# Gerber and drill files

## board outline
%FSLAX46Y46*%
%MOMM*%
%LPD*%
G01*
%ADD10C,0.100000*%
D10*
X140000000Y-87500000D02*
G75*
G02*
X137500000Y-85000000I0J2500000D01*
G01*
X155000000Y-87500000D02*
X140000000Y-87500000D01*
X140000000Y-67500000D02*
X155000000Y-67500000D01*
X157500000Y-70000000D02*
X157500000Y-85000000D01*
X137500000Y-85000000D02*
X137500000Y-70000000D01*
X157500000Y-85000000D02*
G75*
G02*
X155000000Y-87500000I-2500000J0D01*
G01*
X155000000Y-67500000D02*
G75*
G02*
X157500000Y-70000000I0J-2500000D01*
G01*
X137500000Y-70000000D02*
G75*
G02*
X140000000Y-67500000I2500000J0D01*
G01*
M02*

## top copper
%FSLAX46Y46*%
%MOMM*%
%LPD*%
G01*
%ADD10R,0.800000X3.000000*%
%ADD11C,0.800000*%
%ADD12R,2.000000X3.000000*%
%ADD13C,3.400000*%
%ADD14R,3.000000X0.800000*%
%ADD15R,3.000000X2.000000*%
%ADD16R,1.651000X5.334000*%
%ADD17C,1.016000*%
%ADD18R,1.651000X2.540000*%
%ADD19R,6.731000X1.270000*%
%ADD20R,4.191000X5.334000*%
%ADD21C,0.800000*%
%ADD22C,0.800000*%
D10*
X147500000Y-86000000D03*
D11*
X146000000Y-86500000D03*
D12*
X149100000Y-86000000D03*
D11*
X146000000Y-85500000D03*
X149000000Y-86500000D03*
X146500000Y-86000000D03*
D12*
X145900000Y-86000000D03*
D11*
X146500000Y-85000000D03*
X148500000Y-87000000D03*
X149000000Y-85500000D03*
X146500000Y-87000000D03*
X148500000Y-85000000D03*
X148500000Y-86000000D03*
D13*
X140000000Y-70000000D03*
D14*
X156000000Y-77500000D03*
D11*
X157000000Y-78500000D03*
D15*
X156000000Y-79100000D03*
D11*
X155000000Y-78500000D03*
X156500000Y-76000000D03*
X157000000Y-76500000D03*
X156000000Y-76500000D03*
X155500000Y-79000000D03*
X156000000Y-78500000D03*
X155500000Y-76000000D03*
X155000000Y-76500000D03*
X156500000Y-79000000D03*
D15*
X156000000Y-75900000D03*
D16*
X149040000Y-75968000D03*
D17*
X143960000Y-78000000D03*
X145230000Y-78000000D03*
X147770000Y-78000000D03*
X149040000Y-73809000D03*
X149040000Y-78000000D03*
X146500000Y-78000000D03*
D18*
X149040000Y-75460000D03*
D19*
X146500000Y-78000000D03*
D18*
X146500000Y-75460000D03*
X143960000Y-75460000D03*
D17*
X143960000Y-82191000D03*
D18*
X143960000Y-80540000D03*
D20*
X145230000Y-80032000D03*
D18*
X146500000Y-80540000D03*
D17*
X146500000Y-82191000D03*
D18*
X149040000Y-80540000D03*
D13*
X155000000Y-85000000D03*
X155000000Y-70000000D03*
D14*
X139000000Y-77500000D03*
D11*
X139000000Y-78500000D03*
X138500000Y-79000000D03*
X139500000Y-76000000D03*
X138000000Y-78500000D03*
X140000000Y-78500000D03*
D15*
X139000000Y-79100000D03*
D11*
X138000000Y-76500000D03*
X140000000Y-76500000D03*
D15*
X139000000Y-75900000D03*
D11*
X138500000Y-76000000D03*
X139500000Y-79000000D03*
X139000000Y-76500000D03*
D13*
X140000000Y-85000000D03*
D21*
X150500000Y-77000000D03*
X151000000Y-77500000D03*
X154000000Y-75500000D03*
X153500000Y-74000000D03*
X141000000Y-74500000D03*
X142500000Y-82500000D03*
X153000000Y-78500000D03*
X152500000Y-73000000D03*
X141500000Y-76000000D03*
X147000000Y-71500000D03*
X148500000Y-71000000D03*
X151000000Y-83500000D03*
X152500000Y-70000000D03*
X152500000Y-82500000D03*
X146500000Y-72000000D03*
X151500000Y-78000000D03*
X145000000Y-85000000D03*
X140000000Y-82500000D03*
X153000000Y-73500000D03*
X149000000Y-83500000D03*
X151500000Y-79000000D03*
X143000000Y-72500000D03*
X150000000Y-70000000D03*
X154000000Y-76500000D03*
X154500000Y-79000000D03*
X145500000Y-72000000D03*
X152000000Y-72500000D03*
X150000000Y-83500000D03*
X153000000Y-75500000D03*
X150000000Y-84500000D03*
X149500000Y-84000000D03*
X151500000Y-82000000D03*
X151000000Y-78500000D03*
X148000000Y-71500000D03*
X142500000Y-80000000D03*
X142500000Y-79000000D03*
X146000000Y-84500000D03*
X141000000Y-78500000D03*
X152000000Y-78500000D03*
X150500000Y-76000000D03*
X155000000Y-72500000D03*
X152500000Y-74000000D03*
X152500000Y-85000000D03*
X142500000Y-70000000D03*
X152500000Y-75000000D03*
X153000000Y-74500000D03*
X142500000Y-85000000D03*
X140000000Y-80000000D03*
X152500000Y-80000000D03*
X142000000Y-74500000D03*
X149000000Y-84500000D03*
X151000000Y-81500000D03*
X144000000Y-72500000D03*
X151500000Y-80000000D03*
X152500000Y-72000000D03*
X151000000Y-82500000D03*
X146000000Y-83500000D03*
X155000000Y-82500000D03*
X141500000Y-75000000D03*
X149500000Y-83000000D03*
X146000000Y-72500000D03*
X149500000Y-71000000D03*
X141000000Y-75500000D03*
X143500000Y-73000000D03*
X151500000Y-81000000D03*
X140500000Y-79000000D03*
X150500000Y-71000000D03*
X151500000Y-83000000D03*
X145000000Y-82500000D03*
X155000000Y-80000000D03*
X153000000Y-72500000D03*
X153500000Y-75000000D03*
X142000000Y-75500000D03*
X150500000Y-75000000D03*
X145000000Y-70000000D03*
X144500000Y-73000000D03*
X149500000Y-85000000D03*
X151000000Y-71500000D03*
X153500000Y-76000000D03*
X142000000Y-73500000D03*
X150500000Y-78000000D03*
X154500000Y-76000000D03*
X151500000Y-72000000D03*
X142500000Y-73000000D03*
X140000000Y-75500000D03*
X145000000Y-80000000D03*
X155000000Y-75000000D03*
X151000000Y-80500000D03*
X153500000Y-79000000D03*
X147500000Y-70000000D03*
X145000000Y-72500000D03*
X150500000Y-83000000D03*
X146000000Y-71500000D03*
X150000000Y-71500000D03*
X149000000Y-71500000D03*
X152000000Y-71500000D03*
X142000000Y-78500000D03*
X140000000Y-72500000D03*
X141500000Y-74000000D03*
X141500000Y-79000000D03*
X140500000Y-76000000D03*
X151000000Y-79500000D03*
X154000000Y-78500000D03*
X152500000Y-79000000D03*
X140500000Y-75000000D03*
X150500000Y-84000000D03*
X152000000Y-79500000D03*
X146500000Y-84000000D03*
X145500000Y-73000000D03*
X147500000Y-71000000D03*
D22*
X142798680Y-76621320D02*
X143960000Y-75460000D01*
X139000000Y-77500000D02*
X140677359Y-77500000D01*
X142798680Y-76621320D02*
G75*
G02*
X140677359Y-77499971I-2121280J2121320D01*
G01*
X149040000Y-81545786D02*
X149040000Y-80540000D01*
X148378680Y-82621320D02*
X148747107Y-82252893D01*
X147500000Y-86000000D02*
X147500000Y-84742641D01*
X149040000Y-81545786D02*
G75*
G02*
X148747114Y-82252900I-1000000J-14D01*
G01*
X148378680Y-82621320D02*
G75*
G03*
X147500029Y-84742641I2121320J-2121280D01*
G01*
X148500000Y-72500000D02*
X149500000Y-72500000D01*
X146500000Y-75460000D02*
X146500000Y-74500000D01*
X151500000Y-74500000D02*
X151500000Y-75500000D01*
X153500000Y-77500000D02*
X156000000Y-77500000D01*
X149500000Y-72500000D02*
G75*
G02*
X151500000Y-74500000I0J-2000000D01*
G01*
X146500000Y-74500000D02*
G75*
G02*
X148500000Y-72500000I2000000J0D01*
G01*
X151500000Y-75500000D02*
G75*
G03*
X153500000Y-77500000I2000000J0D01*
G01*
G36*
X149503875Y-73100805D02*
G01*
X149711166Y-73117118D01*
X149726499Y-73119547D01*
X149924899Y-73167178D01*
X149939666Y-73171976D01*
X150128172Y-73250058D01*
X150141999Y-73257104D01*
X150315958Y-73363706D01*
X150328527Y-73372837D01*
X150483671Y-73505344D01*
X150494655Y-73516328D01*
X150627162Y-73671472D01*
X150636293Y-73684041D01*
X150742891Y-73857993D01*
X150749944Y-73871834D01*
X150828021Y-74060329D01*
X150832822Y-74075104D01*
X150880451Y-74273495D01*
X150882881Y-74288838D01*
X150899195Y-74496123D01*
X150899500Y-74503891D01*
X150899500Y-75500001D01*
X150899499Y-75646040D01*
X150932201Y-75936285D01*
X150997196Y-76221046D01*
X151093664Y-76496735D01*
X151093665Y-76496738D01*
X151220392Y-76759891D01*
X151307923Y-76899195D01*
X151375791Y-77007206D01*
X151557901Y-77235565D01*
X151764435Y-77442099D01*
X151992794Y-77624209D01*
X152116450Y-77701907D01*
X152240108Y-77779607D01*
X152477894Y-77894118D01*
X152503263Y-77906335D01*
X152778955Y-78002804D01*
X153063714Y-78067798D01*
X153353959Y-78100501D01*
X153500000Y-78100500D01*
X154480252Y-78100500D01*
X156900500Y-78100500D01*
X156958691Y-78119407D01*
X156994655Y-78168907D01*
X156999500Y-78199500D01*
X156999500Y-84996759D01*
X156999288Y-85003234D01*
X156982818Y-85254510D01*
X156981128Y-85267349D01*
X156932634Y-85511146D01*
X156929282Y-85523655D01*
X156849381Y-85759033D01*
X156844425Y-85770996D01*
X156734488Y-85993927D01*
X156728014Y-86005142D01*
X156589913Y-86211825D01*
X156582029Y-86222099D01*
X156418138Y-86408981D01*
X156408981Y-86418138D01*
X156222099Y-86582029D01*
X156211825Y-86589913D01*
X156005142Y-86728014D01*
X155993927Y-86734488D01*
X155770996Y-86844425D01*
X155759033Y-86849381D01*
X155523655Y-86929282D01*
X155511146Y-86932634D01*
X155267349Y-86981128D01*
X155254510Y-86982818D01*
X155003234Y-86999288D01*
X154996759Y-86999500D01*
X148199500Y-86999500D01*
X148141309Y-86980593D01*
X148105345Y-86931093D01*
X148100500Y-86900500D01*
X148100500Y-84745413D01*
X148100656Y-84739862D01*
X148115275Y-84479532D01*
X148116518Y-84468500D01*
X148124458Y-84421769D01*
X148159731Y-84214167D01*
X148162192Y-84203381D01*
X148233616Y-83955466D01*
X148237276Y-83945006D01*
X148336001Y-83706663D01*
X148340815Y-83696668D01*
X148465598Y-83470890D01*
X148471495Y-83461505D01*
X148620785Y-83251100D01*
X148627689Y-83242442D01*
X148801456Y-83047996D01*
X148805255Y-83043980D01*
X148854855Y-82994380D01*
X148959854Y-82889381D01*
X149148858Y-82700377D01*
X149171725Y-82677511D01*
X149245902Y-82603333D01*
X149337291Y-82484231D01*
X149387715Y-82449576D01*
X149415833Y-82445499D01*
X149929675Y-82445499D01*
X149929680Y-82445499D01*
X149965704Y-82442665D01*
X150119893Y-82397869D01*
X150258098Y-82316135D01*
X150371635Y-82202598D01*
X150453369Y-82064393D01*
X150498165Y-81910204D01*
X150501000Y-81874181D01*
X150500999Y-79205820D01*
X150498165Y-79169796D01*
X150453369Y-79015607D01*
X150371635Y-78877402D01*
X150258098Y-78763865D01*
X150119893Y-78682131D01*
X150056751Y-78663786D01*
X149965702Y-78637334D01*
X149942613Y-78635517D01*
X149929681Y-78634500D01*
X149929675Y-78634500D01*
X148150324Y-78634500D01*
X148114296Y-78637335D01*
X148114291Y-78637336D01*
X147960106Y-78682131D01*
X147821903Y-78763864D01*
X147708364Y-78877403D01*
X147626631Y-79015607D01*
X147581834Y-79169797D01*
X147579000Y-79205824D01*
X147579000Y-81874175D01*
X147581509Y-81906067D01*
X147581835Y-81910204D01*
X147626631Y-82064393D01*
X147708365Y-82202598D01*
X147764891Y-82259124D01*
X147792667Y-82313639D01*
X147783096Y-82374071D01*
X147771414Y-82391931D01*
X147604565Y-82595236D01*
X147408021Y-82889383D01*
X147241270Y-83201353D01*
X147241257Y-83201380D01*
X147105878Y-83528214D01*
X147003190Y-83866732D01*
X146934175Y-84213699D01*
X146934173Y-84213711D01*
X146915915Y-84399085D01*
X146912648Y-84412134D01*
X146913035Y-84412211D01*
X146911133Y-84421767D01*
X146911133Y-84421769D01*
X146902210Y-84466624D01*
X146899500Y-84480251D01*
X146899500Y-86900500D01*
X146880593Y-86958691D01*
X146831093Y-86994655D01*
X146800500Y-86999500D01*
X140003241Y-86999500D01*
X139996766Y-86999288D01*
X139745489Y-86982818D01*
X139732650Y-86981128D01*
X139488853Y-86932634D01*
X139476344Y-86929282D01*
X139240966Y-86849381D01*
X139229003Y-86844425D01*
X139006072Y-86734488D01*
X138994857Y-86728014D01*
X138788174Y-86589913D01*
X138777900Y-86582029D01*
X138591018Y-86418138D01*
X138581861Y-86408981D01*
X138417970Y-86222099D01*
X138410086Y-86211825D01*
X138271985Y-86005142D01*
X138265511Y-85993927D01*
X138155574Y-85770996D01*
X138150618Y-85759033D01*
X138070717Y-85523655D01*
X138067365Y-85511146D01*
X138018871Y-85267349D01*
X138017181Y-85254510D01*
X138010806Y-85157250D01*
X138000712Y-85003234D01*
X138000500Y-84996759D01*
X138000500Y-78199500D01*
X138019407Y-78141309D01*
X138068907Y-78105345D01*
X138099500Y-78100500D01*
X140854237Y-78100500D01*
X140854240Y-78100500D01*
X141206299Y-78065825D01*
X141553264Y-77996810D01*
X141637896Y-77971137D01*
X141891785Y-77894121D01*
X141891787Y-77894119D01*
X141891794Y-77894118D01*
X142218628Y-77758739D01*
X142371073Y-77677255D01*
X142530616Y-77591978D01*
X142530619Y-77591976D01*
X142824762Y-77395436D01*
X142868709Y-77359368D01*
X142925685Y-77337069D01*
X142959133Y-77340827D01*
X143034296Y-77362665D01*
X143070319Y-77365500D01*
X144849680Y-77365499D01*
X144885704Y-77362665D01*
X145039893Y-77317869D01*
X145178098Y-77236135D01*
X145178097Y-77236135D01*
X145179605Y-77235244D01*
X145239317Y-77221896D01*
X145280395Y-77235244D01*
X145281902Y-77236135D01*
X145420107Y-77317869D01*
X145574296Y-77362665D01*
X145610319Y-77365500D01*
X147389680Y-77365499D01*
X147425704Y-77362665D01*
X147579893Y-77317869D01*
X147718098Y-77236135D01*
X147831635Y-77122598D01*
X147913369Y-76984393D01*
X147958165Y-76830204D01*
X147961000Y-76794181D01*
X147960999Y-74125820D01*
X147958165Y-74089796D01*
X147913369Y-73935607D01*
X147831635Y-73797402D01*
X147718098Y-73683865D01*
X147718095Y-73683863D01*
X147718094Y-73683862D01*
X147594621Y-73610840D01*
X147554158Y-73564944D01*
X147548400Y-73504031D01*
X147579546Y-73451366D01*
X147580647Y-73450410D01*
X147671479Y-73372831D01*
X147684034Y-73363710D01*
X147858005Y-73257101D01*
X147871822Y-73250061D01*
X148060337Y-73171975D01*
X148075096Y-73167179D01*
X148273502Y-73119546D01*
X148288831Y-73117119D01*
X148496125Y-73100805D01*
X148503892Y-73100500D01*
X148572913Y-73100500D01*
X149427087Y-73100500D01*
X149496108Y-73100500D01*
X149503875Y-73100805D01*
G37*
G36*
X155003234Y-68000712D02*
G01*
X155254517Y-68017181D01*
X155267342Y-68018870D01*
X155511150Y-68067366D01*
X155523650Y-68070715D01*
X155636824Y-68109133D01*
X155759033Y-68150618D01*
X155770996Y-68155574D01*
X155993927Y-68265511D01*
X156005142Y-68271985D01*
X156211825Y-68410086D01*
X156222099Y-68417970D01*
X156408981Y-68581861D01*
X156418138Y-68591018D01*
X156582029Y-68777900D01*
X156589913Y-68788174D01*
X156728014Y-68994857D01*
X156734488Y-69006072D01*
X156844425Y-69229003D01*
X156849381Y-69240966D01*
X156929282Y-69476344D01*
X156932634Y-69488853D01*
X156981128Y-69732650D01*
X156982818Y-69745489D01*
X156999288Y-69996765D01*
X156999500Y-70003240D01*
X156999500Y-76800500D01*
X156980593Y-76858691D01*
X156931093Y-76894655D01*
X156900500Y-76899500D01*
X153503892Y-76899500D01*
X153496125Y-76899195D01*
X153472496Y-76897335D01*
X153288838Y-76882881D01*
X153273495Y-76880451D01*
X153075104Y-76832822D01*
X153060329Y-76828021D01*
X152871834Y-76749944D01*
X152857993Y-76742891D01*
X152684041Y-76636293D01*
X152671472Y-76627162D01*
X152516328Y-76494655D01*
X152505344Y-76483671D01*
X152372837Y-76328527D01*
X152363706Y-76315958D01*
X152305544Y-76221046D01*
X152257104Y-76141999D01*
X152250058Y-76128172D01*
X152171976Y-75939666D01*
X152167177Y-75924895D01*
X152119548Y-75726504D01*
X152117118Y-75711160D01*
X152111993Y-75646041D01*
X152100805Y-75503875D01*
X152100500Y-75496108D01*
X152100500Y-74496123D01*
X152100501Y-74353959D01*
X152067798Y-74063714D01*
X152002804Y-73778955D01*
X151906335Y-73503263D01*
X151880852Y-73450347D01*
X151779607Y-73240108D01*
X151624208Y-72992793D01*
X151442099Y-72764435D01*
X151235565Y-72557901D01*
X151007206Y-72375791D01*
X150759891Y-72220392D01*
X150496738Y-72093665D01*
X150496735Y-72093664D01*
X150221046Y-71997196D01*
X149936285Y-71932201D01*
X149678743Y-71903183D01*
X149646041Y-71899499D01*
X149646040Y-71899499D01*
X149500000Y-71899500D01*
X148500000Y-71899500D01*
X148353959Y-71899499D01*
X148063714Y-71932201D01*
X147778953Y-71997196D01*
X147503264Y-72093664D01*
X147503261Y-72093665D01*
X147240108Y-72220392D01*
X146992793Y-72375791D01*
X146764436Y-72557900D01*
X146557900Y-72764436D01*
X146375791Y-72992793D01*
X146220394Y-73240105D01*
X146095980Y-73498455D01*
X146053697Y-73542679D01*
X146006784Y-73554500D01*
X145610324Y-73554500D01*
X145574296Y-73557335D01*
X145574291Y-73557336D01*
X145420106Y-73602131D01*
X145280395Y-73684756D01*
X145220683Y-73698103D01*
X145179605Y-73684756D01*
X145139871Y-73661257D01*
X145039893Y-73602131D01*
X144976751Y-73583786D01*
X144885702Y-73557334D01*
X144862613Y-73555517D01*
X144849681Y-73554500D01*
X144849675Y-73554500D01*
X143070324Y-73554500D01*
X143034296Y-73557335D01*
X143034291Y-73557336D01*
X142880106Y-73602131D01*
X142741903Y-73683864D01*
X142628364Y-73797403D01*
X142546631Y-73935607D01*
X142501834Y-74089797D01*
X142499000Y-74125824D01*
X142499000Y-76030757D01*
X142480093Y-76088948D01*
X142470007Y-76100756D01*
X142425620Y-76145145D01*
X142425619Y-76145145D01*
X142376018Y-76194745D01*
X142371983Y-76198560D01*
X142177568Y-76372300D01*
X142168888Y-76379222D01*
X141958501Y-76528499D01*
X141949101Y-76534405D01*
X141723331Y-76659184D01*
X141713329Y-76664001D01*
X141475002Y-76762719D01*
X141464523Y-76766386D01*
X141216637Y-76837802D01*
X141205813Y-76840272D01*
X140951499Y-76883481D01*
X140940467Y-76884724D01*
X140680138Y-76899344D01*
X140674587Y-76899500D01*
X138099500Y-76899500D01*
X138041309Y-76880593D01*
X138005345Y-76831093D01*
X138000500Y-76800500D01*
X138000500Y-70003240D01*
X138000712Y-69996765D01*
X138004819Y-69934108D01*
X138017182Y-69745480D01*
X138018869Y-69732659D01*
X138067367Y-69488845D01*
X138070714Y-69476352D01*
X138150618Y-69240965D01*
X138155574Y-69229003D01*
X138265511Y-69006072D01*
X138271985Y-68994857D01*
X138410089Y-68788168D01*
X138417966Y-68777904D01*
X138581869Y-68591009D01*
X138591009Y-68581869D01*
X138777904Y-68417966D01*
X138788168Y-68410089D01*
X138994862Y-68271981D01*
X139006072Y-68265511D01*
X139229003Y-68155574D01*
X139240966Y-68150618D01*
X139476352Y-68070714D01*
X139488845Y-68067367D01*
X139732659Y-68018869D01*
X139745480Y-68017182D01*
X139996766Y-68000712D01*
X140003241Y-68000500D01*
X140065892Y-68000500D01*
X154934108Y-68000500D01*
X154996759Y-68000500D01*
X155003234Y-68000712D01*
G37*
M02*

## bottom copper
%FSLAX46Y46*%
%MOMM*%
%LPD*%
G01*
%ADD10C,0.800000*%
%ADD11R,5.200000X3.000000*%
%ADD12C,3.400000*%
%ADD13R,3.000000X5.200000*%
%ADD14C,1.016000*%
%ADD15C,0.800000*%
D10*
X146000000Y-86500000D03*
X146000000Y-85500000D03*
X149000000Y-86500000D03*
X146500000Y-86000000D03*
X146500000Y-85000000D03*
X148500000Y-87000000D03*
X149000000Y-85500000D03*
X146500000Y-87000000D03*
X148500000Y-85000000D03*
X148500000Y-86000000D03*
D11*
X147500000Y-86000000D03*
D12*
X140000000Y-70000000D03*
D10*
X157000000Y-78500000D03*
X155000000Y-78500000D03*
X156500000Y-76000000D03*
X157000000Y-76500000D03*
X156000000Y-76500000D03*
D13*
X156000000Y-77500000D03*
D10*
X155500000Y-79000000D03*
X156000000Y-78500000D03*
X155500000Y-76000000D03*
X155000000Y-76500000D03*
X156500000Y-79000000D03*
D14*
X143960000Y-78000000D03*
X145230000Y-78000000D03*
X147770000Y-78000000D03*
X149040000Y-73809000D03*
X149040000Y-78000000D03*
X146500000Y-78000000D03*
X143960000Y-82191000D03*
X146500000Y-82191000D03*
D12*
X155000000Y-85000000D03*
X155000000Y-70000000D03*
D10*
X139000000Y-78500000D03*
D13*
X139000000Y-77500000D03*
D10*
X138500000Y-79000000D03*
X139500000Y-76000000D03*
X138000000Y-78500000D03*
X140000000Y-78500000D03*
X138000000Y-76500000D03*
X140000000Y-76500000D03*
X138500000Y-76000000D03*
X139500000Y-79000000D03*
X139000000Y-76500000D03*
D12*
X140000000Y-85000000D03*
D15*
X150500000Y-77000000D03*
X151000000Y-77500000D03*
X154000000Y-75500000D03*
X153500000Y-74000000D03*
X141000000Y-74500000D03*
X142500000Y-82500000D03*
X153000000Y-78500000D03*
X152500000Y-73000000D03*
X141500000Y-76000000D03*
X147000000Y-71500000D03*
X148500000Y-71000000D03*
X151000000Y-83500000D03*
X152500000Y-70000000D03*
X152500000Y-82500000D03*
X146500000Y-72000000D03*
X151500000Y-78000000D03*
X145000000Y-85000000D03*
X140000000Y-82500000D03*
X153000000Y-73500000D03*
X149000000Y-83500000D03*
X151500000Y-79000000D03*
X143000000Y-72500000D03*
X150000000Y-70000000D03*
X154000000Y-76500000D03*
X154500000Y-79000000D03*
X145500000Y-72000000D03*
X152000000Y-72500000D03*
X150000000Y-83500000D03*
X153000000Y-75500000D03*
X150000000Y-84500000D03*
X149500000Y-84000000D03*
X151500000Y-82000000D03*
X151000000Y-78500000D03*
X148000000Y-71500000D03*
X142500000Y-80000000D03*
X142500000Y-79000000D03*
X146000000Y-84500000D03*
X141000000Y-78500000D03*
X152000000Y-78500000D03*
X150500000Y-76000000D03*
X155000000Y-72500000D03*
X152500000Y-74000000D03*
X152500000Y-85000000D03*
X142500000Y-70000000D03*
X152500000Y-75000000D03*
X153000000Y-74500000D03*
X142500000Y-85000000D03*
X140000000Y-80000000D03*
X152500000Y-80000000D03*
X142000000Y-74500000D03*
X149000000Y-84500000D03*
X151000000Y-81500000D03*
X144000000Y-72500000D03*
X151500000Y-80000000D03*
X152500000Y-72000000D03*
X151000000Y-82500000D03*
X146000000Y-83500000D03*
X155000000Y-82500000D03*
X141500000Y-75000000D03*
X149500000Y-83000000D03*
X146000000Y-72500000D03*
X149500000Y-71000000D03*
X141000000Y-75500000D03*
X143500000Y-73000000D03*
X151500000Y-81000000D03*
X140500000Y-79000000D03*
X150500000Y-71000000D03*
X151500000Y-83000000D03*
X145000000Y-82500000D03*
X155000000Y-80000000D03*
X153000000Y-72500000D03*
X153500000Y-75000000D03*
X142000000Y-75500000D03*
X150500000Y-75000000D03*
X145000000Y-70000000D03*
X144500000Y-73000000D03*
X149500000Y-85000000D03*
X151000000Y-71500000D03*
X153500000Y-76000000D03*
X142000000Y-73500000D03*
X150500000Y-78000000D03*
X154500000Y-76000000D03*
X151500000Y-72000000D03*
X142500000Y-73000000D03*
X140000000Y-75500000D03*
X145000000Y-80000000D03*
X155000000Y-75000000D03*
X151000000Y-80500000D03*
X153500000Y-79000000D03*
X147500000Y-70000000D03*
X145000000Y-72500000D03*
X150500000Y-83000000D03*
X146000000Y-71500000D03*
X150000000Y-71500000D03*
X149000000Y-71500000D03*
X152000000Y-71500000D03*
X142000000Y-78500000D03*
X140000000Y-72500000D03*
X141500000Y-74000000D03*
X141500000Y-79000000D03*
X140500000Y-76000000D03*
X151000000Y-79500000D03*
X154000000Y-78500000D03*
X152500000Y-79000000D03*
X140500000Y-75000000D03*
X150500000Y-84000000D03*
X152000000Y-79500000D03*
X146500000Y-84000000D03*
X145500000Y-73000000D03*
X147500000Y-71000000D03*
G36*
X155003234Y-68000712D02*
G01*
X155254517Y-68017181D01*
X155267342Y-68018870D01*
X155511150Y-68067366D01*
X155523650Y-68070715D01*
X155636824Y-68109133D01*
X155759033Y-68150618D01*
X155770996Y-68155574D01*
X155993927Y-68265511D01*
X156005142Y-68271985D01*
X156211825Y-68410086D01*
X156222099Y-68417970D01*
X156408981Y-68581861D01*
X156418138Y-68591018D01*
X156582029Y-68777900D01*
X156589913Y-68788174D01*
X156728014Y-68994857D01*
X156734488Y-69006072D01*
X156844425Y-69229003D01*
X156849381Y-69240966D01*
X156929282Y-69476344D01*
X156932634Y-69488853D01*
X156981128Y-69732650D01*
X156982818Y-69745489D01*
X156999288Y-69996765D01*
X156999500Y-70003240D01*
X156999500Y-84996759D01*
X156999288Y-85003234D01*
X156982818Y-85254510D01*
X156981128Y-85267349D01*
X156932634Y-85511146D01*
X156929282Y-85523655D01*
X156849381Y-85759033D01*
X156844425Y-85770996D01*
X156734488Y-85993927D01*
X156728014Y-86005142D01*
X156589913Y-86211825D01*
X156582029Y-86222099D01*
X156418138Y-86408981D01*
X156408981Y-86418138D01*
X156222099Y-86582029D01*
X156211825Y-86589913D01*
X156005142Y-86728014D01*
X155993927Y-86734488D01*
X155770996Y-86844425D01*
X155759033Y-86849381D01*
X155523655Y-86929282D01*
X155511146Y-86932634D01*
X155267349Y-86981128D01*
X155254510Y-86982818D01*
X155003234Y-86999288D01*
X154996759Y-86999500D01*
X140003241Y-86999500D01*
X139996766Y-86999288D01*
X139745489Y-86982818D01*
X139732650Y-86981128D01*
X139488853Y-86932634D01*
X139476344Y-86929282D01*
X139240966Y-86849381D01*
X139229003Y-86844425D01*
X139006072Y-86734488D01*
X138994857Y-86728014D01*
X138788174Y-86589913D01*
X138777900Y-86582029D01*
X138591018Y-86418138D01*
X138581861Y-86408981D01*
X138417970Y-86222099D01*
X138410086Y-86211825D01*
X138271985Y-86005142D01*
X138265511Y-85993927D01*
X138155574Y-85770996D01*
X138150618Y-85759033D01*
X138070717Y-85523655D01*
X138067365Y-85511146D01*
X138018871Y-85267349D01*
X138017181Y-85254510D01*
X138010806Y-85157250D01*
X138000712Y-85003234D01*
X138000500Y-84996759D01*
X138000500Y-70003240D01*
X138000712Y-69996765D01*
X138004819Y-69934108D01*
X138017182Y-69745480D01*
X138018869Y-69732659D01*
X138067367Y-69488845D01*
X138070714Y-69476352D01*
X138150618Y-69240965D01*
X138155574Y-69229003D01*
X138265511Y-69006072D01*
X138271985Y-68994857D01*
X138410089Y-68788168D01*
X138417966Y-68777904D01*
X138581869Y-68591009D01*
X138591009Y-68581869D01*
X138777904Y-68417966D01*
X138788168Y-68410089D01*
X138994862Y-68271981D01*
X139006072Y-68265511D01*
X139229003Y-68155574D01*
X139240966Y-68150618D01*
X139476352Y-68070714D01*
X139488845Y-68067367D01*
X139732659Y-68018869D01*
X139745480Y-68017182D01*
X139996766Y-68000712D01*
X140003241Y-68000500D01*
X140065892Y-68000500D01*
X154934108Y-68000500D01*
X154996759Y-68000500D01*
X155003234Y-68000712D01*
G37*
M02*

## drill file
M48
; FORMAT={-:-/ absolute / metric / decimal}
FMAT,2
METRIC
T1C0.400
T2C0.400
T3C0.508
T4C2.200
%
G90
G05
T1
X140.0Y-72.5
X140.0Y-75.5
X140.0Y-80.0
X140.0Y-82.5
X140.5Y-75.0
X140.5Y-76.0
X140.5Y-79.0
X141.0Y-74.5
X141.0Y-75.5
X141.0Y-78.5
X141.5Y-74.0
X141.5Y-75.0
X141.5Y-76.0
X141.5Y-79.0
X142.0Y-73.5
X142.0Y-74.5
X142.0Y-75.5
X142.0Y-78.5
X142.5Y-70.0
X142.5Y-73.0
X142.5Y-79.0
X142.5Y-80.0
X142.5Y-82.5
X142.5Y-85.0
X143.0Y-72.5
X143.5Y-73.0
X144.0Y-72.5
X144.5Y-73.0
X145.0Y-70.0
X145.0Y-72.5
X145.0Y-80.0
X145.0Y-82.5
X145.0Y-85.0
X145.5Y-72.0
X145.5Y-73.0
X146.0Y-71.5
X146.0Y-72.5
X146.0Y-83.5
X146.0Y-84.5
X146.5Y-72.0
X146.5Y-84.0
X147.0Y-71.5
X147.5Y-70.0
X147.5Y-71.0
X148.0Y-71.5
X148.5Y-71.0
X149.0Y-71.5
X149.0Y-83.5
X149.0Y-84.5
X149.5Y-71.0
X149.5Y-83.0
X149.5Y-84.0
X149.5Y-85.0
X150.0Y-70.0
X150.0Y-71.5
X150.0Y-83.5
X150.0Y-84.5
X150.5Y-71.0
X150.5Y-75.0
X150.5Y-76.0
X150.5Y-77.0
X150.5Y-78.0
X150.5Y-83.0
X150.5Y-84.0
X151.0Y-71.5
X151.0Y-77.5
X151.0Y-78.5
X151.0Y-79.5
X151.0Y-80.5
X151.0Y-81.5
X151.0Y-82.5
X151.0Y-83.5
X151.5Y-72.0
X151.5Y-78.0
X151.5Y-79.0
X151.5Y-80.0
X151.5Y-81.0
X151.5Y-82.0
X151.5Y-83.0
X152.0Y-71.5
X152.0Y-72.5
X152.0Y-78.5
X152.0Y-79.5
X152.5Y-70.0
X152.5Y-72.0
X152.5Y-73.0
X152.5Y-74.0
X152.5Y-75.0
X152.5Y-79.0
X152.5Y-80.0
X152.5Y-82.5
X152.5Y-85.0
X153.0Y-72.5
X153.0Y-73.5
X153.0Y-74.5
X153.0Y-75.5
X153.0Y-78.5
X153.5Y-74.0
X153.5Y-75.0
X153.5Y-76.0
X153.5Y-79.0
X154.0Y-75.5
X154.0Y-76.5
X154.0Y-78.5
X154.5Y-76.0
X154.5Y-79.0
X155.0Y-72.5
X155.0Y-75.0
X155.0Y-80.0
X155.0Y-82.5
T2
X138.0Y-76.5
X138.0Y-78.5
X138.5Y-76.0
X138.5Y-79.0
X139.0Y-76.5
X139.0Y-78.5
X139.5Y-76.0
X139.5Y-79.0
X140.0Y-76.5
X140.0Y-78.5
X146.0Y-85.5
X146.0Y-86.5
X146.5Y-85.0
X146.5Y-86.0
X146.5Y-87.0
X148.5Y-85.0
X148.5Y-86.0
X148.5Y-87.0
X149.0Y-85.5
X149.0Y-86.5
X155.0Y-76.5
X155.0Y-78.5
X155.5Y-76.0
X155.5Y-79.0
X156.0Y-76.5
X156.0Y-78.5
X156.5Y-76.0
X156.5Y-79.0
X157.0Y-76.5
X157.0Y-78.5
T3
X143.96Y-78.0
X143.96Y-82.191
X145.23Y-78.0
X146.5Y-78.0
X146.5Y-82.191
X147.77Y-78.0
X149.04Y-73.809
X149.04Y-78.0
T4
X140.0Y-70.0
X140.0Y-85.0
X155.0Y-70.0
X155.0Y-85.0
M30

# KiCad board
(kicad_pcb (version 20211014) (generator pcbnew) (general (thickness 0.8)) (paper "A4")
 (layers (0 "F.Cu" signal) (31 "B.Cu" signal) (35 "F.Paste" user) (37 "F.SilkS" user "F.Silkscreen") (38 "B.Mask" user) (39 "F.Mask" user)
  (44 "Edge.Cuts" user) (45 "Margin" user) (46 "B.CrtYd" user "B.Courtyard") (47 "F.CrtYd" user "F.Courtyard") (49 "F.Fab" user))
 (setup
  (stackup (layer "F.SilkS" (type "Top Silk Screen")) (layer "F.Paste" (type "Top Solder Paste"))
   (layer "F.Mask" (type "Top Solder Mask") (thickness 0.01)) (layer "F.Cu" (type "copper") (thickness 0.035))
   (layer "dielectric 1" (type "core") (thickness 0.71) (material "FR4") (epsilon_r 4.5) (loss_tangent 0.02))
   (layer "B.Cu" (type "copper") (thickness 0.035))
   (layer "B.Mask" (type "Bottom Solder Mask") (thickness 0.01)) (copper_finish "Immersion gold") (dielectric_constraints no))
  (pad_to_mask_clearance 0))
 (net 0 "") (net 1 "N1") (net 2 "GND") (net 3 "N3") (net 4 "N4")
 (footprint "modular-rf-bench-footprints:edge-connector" (layer "F.Cu") (at 147.5 87.5 -90)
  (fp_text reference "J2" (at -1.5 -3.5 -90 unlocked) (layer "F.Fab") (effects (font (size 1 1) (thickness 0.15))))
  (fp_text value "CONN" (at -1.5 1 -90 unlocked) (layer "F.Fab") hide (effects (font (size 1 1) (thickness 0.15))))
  (pad "1" smd rect (at -1.5 0 270) (size 3 0.8) (layers "F.Cu") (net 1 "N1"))
  (pad "2" thru_hole circle (at -1 1.5 270) (size 0.8 0.8) (drill 0.4) (layers *.Cu) (remove_unused_layers) (keep_end_layers) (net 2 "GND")
   (zone_connect 2))
  (pad "2" smd rect (at -1.5 -1.6 270) (size 3 2) (layers "F.Cu") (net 2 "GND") (zone_connect 2))
  (pad "2" thru_hole circle (at -2 1.5 270) (size 0.8 0.8) (drill 0.4) (layers *.Cu) (remove_unused_layers) (keep_end_layers) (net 2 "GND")
   (zone_connect 2))
  (pad "2" thru_hole circle (at -1 -1.5 270) (size 0.8 0.8) (drill 0.4) (layers *.Cu) (remove_unused_layers) (keep_end_layers) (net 2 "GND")
   (zone_connect 2))
  (pad "2" thru_hole circle (at -1.5 1 270) (size 0.8 0.8) (drill 0.4) (layers *.Cu) (remove_unused_layers) (keep_end_layers) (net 2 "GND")
   (zone_connect 2))
  (pad "2" smd rect (at -1.5 1.6 270) (size 3 2) (layers "F.Cu") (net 2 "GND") (zone_connect 2))
  (pad "2" thru_hole circle (at -2.5 1 270) (size 0.8 0.8) (drill 0.4) (layers *.Cu) (remove_unused_layers) (keep_end_layers) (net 2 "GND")
   (zone_connect 2))
  (pad "2" thru_hole circle (at -0.5 -1 270) (size 0.8 0.8) (drill 0.4) (layers *.Cu) (remove_unused_layers) (keep_end_layers) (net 2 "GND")
   (zone_connect 2))
  (pad "2" thru_hole circle (at -2 -1.5 270) (size 0.8 0.8) (drill 0.4) (layers *.Cu) (remove_unused_layers) (keep_end_layers) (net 2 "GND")
   (zone_connect 2))
  (pad "2" thru_hole circle (at -0.5 1 270) (size 0.8 0.8) (drill 0.4) (layers *.Cu) (remove_unused_layers) (keep_end_layers) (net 2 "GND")
   (zone_connect 2))
  (pad "2" thru_hole circle (at -2.5 -1 270) (size 0.8 0.8) (drill 0.4) (layers *.Cu) (remove_unused_layers) (keep_end_layers) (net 2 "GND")
   (zone_connect 2))
  (pad "2" thru_hole circle (at -1.5 -1 270) (size 0.8 0.8) (drill 0.4) (layers *.Cu) (remove_unused_layers) (keep_end_layers) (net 2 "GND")
   (zone_connect 2))
  (pad "2" smd rect (at -1.5 0 270) (size 3 5.2) (layers "B.Cu") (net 2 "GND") (zone_connect 2)))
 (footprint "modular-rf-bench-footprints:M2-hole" (layer "F.Cu") (at 140 70)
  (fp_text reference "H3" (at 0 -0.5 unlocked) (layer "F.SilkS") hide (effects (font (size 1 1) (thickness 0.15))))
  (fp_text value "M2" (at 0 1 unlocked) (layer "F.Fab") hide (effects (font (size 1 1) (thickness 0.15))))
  (pad "1" thru_hole circle (at 0 0) (size 3.4 3.4) (drill 2.2) (layers *.Cu *.Mask) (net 2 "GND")))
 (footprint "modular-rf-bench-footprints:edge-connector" (layer "F.Cu") (at 157.5 77.5)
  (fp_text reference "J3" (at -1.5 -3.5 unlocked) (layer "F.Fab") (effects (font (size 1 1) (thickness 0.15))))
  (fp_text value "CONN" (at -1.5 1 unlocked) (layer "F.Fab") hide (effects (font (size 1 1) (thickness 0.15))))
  (pad "1" smd rect (at -1.5 0) (size 3 0.8) (layers "F.Cu") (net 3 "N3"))
  (pad "2" thru_hole circle (at -0.5 1) (size 0.8 0.8) (drill 0.4) (layers *.Cu) (remove_unused_layers) (keep_end_layers) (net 2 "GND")
   (zone_connect 2))
  (pad "2" smd rect (at -1.5 1.6) (size 3 2) (layers "F.Cu") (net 2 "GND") (zone_connect 2))
  (pad "2" thru_hole circle (at -2.5 1) (size 0.8 0.8) (drill 0.4) (layers *.Cu) (remove_unused_layers) (keep_end_layers) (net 2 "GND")
   (zone_connect 2))
  (pad "2" thru_hole circle (at -1 -1.5) (size 0.8 0.8) (drill 0.4) (layers *.Cu) (remove_unused_layers) (keep_end_layers) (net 2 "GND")
   (zone_connect 2))
  (pad "2" thru_hole circle (at -0.5 -1) (size 0.8 0.8) (drill 0.4) (layers *.Cu) (remove_unused_layers) (keep_end_layers) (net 2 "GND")
   (zone_connect 2))
  (pad "2" thru_hole circle (at -1.5 -1) (size 0.8 0.8) (drill 0.4) (layers *.Cu) (remove_unused_layers) (keep_end_layers) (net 2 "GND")
   (zone_connect 2))
  (pad "2" smd rect (at -1.5 0) (size 3 5.2) (layers "B.Cu") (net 2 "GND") (zone_connect 2))
  (pad "2" thru_hole circle (at -2 1.5) (size 0.8 0.8) (drill 0.4) (layers *.Cu) (remove_unused_layers) (keep_end_layers) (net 2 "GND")
   (zone_connect 2))
  (pad "2" thru_hole circle (at -1.5 1) (size 0.8 0.8) (drill 0.4) (layers *.Cu) (remove_unused_layers) (keep_end_layers) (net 2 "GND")
   (zone_connect 2))
  (pad "2" thru_hole circle (at -2 -1.5) (size 0.8 0.8) (drill 0.4) (layers *.Cu) (remove_unused_layers) (keep_end_layers) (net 2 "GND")
   (zone_connect 2))
  (pad "2" thru_hole circle (at -2.5 -1) (size 0.8 0.8) (drill 0.4) (layers *.Cu) (remove_unused_layers) (keep_end_layers) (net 2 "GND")
   (zone_connect 2))
  (pad "2" thru_hole circle (at -1 1.5) (size 0.8 0.8) (drill 0.4) (layers *.Cu) (remove_unused_layers) (keep_end_layers) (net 2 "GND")
   (zone_connect 2))
  (pad "2" smd rect (at -1.5 -1.6) (size 3 2) (layers "F.Cu") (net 2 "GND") (zone_connect 2)))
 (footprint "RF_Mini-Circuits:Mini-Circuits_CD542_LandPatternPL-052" (layer "F.Cu") (at 146.5 78 -90)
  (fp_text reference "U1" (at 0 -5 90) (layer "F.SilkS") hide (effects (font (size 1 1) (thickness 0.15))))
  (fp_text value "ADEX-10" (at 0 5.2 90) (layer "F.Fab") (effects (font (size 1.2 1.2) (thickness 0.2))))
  (pad "1" smd rect (at -2.032 -2.54 270) (size 5.334 1.651) (layers "F.Cu") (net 2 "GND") (zone_connect 2))
  (pad "1" thru_hole circle (at 0 2.54 270) (size 1.016 1.016) (drill 0.508) (layers *.Cu) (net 2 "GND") (zone_connect 2))
  (pad "1" thru_hole circle (at 0 1.27 270) (size 1.016 1.016) (drill 0.508) (layers *.Cu) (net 2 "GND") (zone_connect 2))
  (pad "1" thru_hole circle (at 0 -1.27 270) (size 1.016 1.016) (drill 0.508) (layers *.Cu) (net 2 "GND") (zone_connect 2))
  (pad "1" thru_hole circle (at -4.191 -2.54 270) (size 1.016 1.016) (drill 0.508) (layers *.Cu) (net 2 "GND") (zone_connect 2))
  (pad "1" thru_hole circle (at 0 -2.54 270) (size 1.016 1.016) (drill 0.508) (layers *.Cu) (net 2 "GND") (zone_connect 2))
  (pad "1" thru_hole circle (at 0 0 270) (size 1.016 1.016) (drill 0.508) (layers *.Cu) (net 2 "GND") (zone_connect 2))
  (pad "1" smd rect (at -2.54 -2.54 270) (size 2.54 1.651) (layers "F.Cu" "F.Paste" "F.Mask") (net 2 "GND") (zone_connect 2))
  (pad "1" smd rect (at 0 0 270) (size 1.27 6.731) (layers "F.Cu") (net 2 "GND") (zone_connect 2))
  (pad "2" smd rect (at -2.54 0 270) (size 2.54 1.651) (layers "F.Cu" "F.Paste" "F.Mask") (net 3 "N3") (clearance 0.635))
  (pad "3" smd rect (at -2.54 2.54 270) (size 2.54 1.651) (layers "F.Cu" "F.Paste" "F.Mask") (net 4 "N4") (clearance 0.635))
  (pad "4" thru_hole circle (at 4.191 2.54 270) (size 1.016 1.016) (drill 0.508) (layers *.Cu) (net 2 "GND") (zone_connect 2))
  (pad "4" smd rect (at 2.54 2.54 270) (size 2.54 1.651) (layers "F.Cu" "F.Paste" "F.Mask") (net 2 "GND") (zone_connect 2))
  (pad "4" smd rect (at 2.032 1.27 270) (size 5.334 4.191) (layers "F.Cu") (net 2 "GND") (zone_connect 2))
  (pad "5" smd rect (at 2.54 0 270) (size 2.54 1.651) (layers "F.Cu" "F.Paste" "F.Mask") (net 2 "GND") (zone_connect 2))
  (pad "5" thru_hole circle (at 4.191 0 270) (size 1.016 1.016) (drill 0.508) (layers *.Cu) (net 2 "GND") (zone_connect 2))
  (pad "6" smd rect (at 2.54 -2.54 270) (size 2.54 1.651) (layers "F.Cu" "F.Paste" "F.Mask") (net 1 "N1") (clearance 0.635)))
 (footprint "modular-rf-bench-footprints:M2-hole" (layer "F.Cu") (at 155 85)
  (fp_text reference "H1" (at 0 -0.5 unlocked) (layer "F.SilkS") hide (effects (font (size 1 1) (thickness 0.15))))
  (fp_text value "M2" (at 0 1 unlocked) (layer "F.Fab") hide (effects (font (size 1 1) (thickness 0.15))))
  (pad "1" thru_hole circle (at 0 0) (size 3.4 3.4) (drill 2.2) (layers *.Cu *.Mask) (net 2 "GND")))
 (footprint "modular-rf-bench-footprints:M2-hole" (layer "F.Cu") (at 155 70)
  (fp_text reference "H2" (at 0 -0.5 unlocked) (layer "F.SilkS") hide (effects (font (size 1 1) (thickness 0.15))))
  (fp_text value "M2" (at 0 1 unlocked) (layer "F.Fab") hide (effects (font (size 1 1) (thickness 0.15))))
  (pad "1" thru_hole circle (at 0 0) (size 3.4 3.4) (drill 2.2) (layers *.Cu *.Mask) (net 2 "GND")))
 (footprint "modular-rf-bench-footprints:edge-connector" (layer "F.Cu") (at 137.5 77.5 180)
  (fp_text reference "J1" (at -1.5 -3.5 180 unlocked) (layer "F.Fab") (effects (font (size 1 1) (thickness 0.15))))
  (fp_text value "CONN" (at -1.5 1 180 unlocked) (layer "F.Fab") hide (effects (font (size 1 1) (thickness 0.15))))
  (pad "1" smd rect (at -1.5 0 180) (size 3 0.8) (layers "F.Cu") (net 4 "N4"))
  (pad "2" thru_hole circle (at -1.5 -1 180) (size 0.8 0.8) (drill 0.4) (layers *.Cu) (remove_unused_layers) (keep_end_layers) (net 2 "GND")
   (zone_connect 2))
  (pad "2" smd rect (at -1.5 0 180) (size 3 5.2) (layers "B.Cu") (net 2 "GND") (zone_connect 2))
  (pad "2" thru_hole circle (at -1 -1.5 180) (size 0.8 0.8) (drill 0.4) (layers *.Cu) (remove_unused_layers) (keep_end_layers) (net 2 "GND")
   (zone_connect 2))
  (pad "2" thru_hole circle (at -2 1.5 180) (size 0.8 0.8) (drill 0.4) (layers *.Cu) (remove_unused_layers) (keep_end_layers) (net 2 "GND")
   (zone_connect 2))
  (pad "2" thru_hole circle (at -0.5 -1 180) (size 0.8 0.8) (drill 0.4) (layers *.Cu) (remove_unused_layers) (keep_end_layers) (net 2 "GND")
   (zone_connect 2))
  (pad "2" thru_hole circle (at -2.5 -1 180) (size 0.8 0.8) (drill 0.4) (layers *.Cu) (remove_unused_layers) (keep_end_layers) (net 2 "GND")
   (zone_connect 2))
  (pad "2" smd rect (at -1.5 -1.6 180) (size 3 2) (layers "F.Cu") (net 2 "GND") (zone_connect 2))
  (pad "2" thru_hole circle (at -0.5 1 180) (size 0.8 0.8) (drill 0.4) (layers *.Cu) (remove_unused_layers) (keep_end_layers) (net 2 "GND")
   (zone_connect 2))
  (pad "2" thru_hole circle (at -2.5 1 180) (size 0.8 0.8) (drill 0.4) (layers *.Cu) (remove_unused_layers) (keep_end_layers) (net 2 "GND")
   (zone_connect 2))
  (pad "2" smd rect (at -1.5 1.6 180) (size 3 2) (layers "F.Cu") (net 2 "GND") (zone_connect 2))
  (pad "2" thru_hole circle (at -1 1.5 180) (size 0.8 0.8) (drill 0.4) (layers *.Cu) (remove_unused_layers) (keep_end_layers) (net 2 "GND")
   (zone_connect 2))
  (pad "2" thru_hole circle (at -2 -1.5 180) (size 0.8 0.8) (drill 0.4) (layers *.Cu) (remove_unused_layers) (keep_end_layers) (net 2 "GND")
   (zone_connect 2))
  (pad "2" thru_hole circle (at -1.5 1 180) (size 0.8 0.8) (drill 0.4) (layers *.Cu) (remove_unused_layers) (keep_end_layers) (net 2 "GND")
   (zone_connect 2)))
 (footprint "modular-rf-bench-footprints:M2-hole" (layer "F.Cu") (at 140 85)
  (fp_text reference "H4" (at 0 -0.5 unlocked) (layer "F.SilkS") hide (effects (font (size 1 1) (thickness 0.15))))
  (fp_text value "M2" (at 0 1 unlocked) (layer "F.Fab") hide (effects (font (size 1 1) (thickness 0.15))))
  (pad "1" thru_hole circle (at 0 0) (size 3.4 3.4) (drill 2.2) (layers *.Cu *.Mask) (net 2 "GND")))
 (gr_arc (start 140 87.5) (mid 138.232233 86.767767) (end 137.5 85) (layer "Edge.Cuts") (width 0.1))
 (gr_line (start 155 87.5) (end 140 87.5) (layer "Edge.Cuts") (width 0.1))
 (gr_line (start 140 67.5) (end 155 67.5) (layer "Edge.Cuts") (width 0.1))
 (gr_line (start 157.5 70) (end 157.5 85) (layer "Edge.Cuts") (width 0.1))
 (gr_line (start 137.5 85) (end 137.5 70) (layer "Edge.Cuts") (width 0.1))
 (gr_arc (start 157.5 85) (mid 156.767767 86.767767) (end 155 87.5) (layer "Edge.Cuts") (width 0.1))
 (gr_arc (start 155 67.5) (mid 156.767767 68.232233) (end 157.5 70) (layer "Edge.Cuts") (width 0.1))
 (gr_arc (start 137.5 70) (mid 138.232233 68.232233) (end 140 67.5) (layer "Edge.Cuts") (width 0.1))
 (via (at 150.5 77) (size 0.8) (drill 0.4) (layers "F.Cu" "B.Cu") (free) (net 2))
 (via (at 151 77.5) (size 0.8) (drill 0.4) (layers "F.Cu" "B.Cu") (free) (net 2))
 (via (at 154 75.5) (size 0.8) (drill 0.4) (layers "F.Cu" "B.Cu") (free) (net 2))
 (via (at 153.5 74) (size 0.8) (drill 0.4) (layers "F.Cu" "B.Cu") (free) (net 2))
 (via (at 141 74.5) (size 0.8) (drill 0.4) (layers "F.Cu" "B.Cu") (free) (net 2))
 (via (at 142.5 82.5) (size 0.8) (drill 0.4) (layers "F.Cu" "B.Cu") (free) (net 2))
 (via (at 153 78.5) (size 0.8) (drill 0.4) (layers "F.Cu" "B.Cu") (free) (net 2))
 (via (at 152.5 73) (size 0.8) (drill 0.4) (layers "F.Cu" "B.Cu") (free) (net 2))
 (via (at 141.5 76) (size 0.8) (drill 0.4) (layers "F.Cu" "B.Cu") (free) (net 2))
 (via (at 147 71.5) (size 0.8) (drill 0.4) (layers "F.Cu" "B.Cu") (free) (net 2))
 (via (at 148.5 71) (size 0.8) (drill 0.4) (layers "F.Cu" "B.Cu") (free) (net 2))
 (via (at 151 83.5) (size 0.8) (drill 0.4) (layers "F.Cu" "B.Cu") (free) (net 2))
 (via (at 152.5 70) (size 0.8) (drill 0.4) (layers "F.Cu" "B.Cu") (free) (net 2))
 (via (at 152.5 82.5) (size 0.8) (drill 0.4) (layers "F.Cu" "B.Cu") (free) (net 2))
 (via (at 146.5 72) (size 0.8) (drill 0.4) (layers "F.Cu" "B.Cu") (free) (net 2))
 (via (at 151.5 78) (size 0.8) (drill 0.4) (layers "F.Cu" "B.Cu") (free) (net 2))
 (via (at 145 85) (size 0.8) (drill 0.4) (layers "F.Cu" "B.Cu") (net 2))
 (via (at 140 82.5) (size 0.8) (drill 0.4) (layers "F.Cu" "B.Cu") (free) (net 2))
 (via (at 153 73.5) (size 0.8) (drill 0.4) (layers "F.Cu" "B.Cu") (free) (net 2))
 (via (at 149 83.5) (size 0.8) (drill 0.4) (layers "F.Cu" "B.Cu") (free) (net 2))
 (via (at 151.5 79) (size 0.8) (drill 0.4) (layers "F.Cu" "B.Cu") (free) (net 2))
 (via (at 143 72.5) (size 0.8) (drill 0.4) (layers "F.Cu" "B.Cu") (free) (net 2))
 (via (at 150 70) (size 0.8) (drill 0.4) (layers "F.Cu" "B.Cu") (free) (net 2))
 (via (at 154 76.5) (size 0.8) (drill 0.4) (layers "F.Cu" "B.Cu") (free) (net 2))
 (via (at 154.5 79) (size 0.8) (drill 0.4) (layers "F.Cu" "B.Cu") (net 2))
 (via (at 145.5 72) (size 0.8) (drill 0.4) (layers "F.Cu" "B.Cu") (free) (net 2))
 (via (at 152 72.5) (size 0.8) (drill 0.4) (layers "F.Cu" "B.Cu") (free) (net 2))
 (via (at 150 83.5) (size 0.8) (drill 0.4) (layers "F.Cu" "B.Cu") (free) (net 2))
 (via (at 153 75.5) (size 0.8) (drill 0.4) (layers "F.Cu" "B.Cu") (free) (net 2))
 (via (at 150 84.5) (size 0.8) (drill 0.4) (layers "F.Cu" "B.Cu") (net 2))
 (via (at 149.5 84) (size 0.8) (drill 0.4) (layers "F.Cu" "B.Cu") (free) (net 2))
 (via (at 151.5 82) (size 0.8) (drill 0.4) (layers "F.Cu" "B.Cu") (free) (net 2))
 (via (at 151 78.5) (size 0.8) (drill 0.4) (layers "F.Cu" "B.Cu") (free) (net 2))
 (via (at 148 71.5) (size 0.8) (drill 0.4) (layers "F.Cu" "B.Cu") (free) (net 2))
 (via (at 142.5 80) (size 0.8) (drill 0.4) (layers "F.Cu" "B.Cu") (free) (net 2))
 (via (at 142.5 79) (size 0.8) (drill 0.4) (layers "F.Cu" "B.Cu") (free) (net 2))
 (via (at 146 84.5) (size 0.8) (drill 0.4) (layers "F.Cu" "B.Cu") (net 2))
 (via (at 141 78.5) (size 0.8) (drill 0.4) (layers "F.Cu" "B.Cu") (free) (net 2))
 (via (at 152 78.5) (size 0.8) (drill 0.4) (layers "F.Cu" "B.Cu") (free) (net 2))
 (via (at 150.5 76) (size 0.8) (drill 0.4) (layers "F.Cu" "B.Cu") (free) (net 2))
 (via (at 155 72.5) (size 0.8) (drill 0.4) (layers "F.Cu" "B.Cu") (free) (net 2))
 (via (at 152.5 74) (size 0.8) (drill 0.4) (layers "F.Cu" "B.Cu") (free) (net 2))
 (via (at 152.5 85) (size 0.8) (drill 0.4) (layers "F.Cu" "B.Cu") (free) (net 2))
 (via (at 142.5 70) (size 0.8) (drill 0.4) (layers "F.Cu" "B.Cu") (free) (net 2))
 (via (at 152.5 75) (size 0.8) (drill 0.4) (layers "F.Cu" "B.Cu") (free) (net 2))
 (via (at 153 74.5) (size 0.8) (drill 0.4) (layers "F.Cu" "B.Cu") (free) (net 2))
 (via (at 142.5 85) (size 0.8) (drill 0.4) (layers "F.Cu" "B.Cu") (free) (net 2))
 (via (at 140 80) (size 0.8) (drill 0.4) (layers "F.Cu" "B.Cu") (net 2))
 (via (at 152.5 80) (size 0.8) (drill 0.4) (layers "F.Cu" "B.Cu") (free) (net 2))
 (via (at 142 74.5) (size 0.8) (drill 0.4) (layers "F.Cu" "B.Cu") (free) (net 2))
 (via (at 149 84.5) (size 0.8) (drill 0.4) (layers "F.Cu" "B.Cu") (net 2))
 (via (at 151 81.5) (size 0.8) (drill 0.4) (layers "F.Cu" "B.Cu") (free) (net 2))
 (via (at 144 72.5) (size 0.8) (drill 0.4) (layers "F.Cu" "B.Cu") (free) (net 2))
 (via (at 151.5 80) (size 0.8) (drill 0.4) (layers "F.Cu" "B.Cu") (free) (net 2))
 (via (at 152.5 72) (size 0.8) (drill 0.4) (layers "F.Cu" "B.Cu") (free) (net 2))
 (via (at 151 82.5) (size 0.8) (drill 0.4) (layers "F.Cu" "B.Cu") (free) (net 2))
 (via (at 146 83.5) (size 0.8) (drill 0.4) (layers "F.Cu" "B.Cu") (free) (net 2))
 (via (at 155 82.5) (size 0.8) (drill 0.4) (layers "F.Cu" "B.Cu") (free) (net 2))
 (via (at 141.5 75) (size 0.8) (drill 0.4) (layers "F.Cu" "B.Cu") (free) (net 2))
 (via (at 149.5 83) (size 0.8) (drill 0.4) (layers "F.Cu" "B.Cu") (free) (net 2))
 (via (at 146 72.5) (size 0.8) (drill 0.4) (layers "F.Cu" "B.Cu") (free) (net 2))
 (via (at 149.5 71) (size 0.8) (drill 0.4) (layers "F.Cu" "B.Cu") (free) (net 2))
 (via (at 141 75.5) (size 0.8) (drill 0.4) (layers "F.Cu" "B.Cu") (free) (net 2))
 (via (at 143.5 73) (size 0.8) (drill 0.4) (layers "F.Cu" "B.Cu") (free) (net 2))
 (via (at 151.5 81) (size 0.8) (drill 0.4) (layers "F.Cu" "B.Cu") (free) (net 2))
 (via (at 140.5 79) (size 0.8) (drill 0.4) (layers "F.Cu" "B.Cu") (free) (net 2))
 (via (at 150.5 71) (size 0.8) (drill 0.4) (layers "F.Cu" "B.Cu") (free) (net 2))
 (via (at 151.5 83) (size 0.8) (drill 0.4) (layers "F.Cu" "B.Cu") (free) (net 2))
 (via (at 145 82.5) (size 0.8) (drill 0.4) (layers "F.Cu" "B.Cu") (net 2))
 (via (at 155 80) (size 0.8) (drill 0.4) (layers "F.Cu" "B.Cu") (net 2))
 (via (at 153 72.5) (size 0.8) (drill 0.4) (layers "F.Cu" "B.Cu") (free) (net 2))
 (via (at 153.5 75) (size 0.8) (drill 0.4) (layers "F.Cu" "B.Cu") (free) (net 2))
 (via (at 142 75.5) (size 0.8) (drill 0.4) (layers "F.Cu" "B.Cu") (free) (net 2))
 (via (at 150.5 75) (size 0.8) (drill 0.4) (layers "F.Cu" "B.Cu") (free) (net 2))
 (via (at 145 70) (size 0.8) (drill 0.4) (layers "F.Cu" "B.Cu") (free) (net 2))
 (via (at 144.5 73) (size 0.8) (drill 0.4) (layers "F.Cu" "B.Cu") (free) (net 2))
 (via (at 149.5 85) (size 0.8) (drill 0.4) (layers "F.Cu" "B.Cu") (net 2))
 (via (at 151 71.5) (size 0.8) (drill 0.4) (layers "F.Cu" "B.Cu") (free) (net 2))
 (via (at 153.5 76) (size 0.8) (drill 0.4) (layers "F.Cu" "B.Cu") (free) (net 2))
 (via (at 142 73.5) (size 0.8) (drill 0.4) (layers "F.Cu" "B.Cu") (free) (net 2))
 (via (at 150.5 78) (size 0.8) (drill 0.4) (layers "F.Cu" "B.Cu") (free) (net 2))
 (via (at 154.5 76) (size 0.8) (drill 0.4) (layers "F.Cu" "B.Cu") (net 2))
 (via (at 151.5 72) (size 0.8) (drill 0.4) (layers "F.Cu" "B.Cu") (free) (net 2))
 (via (at 142.5 73) (size 0.8) (drill 0.4) (layers "F.Cu" "B.Cu") (free) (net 2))
 (via (at 140 75.5) (size 0.8) (drill 0.4) (layers "F.Cu" "B.Cu") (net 2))
 (via (at 145 80) (size 0.8) (drill 0.4) (layers "F.Cu" "B.Cu") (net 2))
 (via (at 155 75) (size 0.8) (drill 0.4) (layers "F.Cu" "B.Cu") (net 2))
 (via (at 151 80.5) (size 0.8) (drill 0.4) (layers "F.Cu" "B.Cu") (free) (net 2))
 (via (at 153.5 79) (size 0.8) (drill 0.4) (layers "F.Cu" "B.Cu") (free) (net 2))
 (via (at 147.5 70) (size 0.8) (drill 0.4) (layers "F.Cu" "B.Cu") (free) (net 2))
 (via (at 145 72.5) (size 0.8) (drill 0.4) (layers "F.Cu" "B.Cu") (free) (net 2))
 (via (at 150.5 83) (size 0.8) (drill 0.4) (layers "F.Cu" "B.Cu") (free) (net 2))
 (via (at 146 71.5) (size 0.8) (drill 0.4) (layers "F.Cu" "B.Cu") (free) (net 2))
 (via (at 150 71.5) (size 0.8) (drill 0.4) (layers "F.Cu" "B.Cu") (free) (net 2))
 (via (at 149 71.5) (size 0.8) (drill 0.4) (layers "F.Cu" "B.Cu") (free) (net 2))
 (via (at 152 71.5) (size 0.8) (drill 0.4) (layers "F.Cu" "B.Cu") (free) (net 2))
 (via (at 142 78.5) (size 0.8) (drill 0.4) (layers "F.Cu" "B.Cu") (free) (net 2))
 (via (at 140 72.5) (size 0.8) (drill 0.4) (layers "F.Cu" "B.Cu") (free) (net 2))
 (via (at 141.5 74) (size 0.8) (drill 0.4) (layers "F.Cu" "B.Cu") (free) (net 2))
 (via (at 141.5 79) (size 0.8) (drill 0.4) (layers "F.Cu" "B.Cu") (free) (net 2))
 (via (at 140.5 76) (size 0.8) (drill 0.4) (layers "F.Cu" "B.Cu") (free) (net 2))
 (via (at 151 79.5) (size 0.8) (drill 0.4) (layers "F.Cu" "B.Cu") (free) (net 2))
 (via (at 154 78.5) (size 0.8) (drill 0.4) (layers "F.Cu" "B.Cu") (free) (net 2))
 (via (at 152.5 79) (size 0.8) (drill 0.4) (layers "F.Cu" "B.Cu") (free) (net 2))
 (via (at 140.5 75) (size 0.8) (drill 0.4) (layers "F.Cu" "B.Cu") (free) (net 2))
 (via (at 150.5 84) (size 0.8) (drill 0.4) (layers "F.Cu" "B.Cu") (free) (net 2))
 (via (at 152 79.5) (size 0.8) (drill 0.4) (layers "F.Cu" "B.Cu") (free) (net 2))
 (via (at 146.5 84) (size 0.8) (drill 0.4) (layers "F.Cu" "B.Cu") (free) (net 2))
 (via (at 145.5 73) (size 0.8) (drill 0.4) (layers "F.Cu" "B.Cu") (free) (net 2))
 (via (at 147.5 71) (size 0.8) (drill 0.4) (layers "F.Cu" "B.Cu") (free) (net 2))
 (segment (start 142.79868 76.62132) (end 143.96 75.46) (width 0.8) (layer "F.Cu") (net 4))
 (segment (start 139 77.5) (end 140.677359 77.5) (width 0.8) (layer "F.Cu") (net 4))
 (arc (start 142.79868 76.62132) (mid 141.82541 77.271639) (end 140.677359 77.5) (width 0.8) (layer "F.Cu") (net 4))
 (segment (start 149.04 81.545786) (end 149.04 80.54) (width 0.8) (layer "F.Cu") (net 1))
 (segment (start 148.37868 82.62132) (end 148.747107 82.252893) (width 0.8) (layer "F.Cu") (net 1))
 (segment (start 147.5 86) (end 147.5 84.742641) (width 0.8) (layer "F.Cu") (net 1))
 (arc (start 149.04 81.545786) (mid 148.96388 81.928469) (end 148.747107 82.252893) (width 0.8) (layer "F.Cu") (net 1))
 (arc (start 148.37868 82.62132) (mid 147.728361 83.59459) (end 147.5 84.742641) (width 0.8) (layer "F.Cu") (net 1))
 (segment (start 148.5 72.5) (end 149.5 72.5) (width 0.8) (layer "F.Cu") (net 3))
 (segment (start 146.5 75.46) (end 146.5 74.5) (width 0.8) (layer "F.Cu") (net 3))
 (segment (start 151.5 74.5) (end 151.5 75.5) (width 0.8) (layer "F.Cu") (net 3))
 (segment (start 153.5 77.5) (end 156 77.5) (width 0.8) (layer "F.Cu") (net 3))
 (arc (start 149.5 72.5) (mid 150.914214 73.085786) (end 151.5 74.5) (width 0.8) (layer "F.Cu") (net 3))
 (arc (start 146.5 74.5) (mid 147.085786 73.085786) (end 148.5 72.5) (width 0.8) (layer "F.Cu") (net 3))
 (arc (start 151.5 75.5) (mid 152.085786 76.914214) (end 153.5 77.5) (width 0.8) (layer "F.Cu") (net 3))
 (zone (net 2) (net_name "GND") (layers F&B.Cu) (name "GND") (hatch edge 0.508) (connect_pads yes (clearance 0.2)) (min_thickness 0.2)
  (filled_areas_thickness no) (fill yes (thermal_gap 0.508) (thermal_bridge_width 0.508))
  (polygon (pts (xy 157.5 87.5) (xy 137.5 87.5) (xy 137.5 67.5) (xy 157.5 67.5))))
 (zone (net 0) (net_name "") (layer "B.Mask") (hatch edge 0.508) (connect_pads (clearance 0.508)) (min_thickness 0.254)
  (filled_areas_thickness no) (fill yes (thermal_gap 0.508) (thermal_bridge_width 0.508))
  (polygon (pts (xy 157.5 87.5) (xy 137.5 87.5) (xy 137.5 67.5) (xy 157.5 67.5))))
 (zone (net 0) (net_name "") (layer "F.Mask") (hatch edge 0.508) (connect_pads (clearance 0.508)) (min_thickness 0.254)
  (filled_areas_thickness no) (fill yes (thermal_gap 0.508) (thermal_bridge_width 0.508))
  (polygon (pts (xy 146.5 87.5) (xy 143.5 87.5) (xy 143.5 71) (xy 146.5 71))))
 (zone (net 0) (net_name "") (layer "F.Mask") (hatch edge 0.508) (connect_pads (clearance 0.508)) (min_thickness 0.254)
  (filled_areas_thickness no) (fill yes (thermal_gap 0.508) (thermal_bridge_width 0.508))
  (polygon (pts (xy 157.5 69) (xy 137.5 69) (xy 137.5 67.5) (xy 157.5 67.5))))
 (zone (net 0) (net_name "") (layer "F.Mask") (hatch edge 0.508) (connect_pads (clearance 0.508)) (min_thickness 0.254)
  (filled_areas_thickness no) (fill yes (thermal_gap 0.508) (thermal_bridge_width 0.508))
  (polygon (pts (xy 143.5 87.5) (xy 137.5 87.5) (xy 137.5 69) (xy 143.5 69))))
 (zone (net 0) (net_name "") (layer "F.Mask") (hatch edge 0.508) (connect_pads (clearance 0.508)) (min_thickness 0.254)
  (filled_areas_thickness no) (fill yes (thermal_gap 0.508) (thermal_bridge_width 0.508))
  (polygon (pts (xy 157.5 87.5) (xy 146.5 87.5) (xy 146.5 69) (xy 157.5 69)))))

